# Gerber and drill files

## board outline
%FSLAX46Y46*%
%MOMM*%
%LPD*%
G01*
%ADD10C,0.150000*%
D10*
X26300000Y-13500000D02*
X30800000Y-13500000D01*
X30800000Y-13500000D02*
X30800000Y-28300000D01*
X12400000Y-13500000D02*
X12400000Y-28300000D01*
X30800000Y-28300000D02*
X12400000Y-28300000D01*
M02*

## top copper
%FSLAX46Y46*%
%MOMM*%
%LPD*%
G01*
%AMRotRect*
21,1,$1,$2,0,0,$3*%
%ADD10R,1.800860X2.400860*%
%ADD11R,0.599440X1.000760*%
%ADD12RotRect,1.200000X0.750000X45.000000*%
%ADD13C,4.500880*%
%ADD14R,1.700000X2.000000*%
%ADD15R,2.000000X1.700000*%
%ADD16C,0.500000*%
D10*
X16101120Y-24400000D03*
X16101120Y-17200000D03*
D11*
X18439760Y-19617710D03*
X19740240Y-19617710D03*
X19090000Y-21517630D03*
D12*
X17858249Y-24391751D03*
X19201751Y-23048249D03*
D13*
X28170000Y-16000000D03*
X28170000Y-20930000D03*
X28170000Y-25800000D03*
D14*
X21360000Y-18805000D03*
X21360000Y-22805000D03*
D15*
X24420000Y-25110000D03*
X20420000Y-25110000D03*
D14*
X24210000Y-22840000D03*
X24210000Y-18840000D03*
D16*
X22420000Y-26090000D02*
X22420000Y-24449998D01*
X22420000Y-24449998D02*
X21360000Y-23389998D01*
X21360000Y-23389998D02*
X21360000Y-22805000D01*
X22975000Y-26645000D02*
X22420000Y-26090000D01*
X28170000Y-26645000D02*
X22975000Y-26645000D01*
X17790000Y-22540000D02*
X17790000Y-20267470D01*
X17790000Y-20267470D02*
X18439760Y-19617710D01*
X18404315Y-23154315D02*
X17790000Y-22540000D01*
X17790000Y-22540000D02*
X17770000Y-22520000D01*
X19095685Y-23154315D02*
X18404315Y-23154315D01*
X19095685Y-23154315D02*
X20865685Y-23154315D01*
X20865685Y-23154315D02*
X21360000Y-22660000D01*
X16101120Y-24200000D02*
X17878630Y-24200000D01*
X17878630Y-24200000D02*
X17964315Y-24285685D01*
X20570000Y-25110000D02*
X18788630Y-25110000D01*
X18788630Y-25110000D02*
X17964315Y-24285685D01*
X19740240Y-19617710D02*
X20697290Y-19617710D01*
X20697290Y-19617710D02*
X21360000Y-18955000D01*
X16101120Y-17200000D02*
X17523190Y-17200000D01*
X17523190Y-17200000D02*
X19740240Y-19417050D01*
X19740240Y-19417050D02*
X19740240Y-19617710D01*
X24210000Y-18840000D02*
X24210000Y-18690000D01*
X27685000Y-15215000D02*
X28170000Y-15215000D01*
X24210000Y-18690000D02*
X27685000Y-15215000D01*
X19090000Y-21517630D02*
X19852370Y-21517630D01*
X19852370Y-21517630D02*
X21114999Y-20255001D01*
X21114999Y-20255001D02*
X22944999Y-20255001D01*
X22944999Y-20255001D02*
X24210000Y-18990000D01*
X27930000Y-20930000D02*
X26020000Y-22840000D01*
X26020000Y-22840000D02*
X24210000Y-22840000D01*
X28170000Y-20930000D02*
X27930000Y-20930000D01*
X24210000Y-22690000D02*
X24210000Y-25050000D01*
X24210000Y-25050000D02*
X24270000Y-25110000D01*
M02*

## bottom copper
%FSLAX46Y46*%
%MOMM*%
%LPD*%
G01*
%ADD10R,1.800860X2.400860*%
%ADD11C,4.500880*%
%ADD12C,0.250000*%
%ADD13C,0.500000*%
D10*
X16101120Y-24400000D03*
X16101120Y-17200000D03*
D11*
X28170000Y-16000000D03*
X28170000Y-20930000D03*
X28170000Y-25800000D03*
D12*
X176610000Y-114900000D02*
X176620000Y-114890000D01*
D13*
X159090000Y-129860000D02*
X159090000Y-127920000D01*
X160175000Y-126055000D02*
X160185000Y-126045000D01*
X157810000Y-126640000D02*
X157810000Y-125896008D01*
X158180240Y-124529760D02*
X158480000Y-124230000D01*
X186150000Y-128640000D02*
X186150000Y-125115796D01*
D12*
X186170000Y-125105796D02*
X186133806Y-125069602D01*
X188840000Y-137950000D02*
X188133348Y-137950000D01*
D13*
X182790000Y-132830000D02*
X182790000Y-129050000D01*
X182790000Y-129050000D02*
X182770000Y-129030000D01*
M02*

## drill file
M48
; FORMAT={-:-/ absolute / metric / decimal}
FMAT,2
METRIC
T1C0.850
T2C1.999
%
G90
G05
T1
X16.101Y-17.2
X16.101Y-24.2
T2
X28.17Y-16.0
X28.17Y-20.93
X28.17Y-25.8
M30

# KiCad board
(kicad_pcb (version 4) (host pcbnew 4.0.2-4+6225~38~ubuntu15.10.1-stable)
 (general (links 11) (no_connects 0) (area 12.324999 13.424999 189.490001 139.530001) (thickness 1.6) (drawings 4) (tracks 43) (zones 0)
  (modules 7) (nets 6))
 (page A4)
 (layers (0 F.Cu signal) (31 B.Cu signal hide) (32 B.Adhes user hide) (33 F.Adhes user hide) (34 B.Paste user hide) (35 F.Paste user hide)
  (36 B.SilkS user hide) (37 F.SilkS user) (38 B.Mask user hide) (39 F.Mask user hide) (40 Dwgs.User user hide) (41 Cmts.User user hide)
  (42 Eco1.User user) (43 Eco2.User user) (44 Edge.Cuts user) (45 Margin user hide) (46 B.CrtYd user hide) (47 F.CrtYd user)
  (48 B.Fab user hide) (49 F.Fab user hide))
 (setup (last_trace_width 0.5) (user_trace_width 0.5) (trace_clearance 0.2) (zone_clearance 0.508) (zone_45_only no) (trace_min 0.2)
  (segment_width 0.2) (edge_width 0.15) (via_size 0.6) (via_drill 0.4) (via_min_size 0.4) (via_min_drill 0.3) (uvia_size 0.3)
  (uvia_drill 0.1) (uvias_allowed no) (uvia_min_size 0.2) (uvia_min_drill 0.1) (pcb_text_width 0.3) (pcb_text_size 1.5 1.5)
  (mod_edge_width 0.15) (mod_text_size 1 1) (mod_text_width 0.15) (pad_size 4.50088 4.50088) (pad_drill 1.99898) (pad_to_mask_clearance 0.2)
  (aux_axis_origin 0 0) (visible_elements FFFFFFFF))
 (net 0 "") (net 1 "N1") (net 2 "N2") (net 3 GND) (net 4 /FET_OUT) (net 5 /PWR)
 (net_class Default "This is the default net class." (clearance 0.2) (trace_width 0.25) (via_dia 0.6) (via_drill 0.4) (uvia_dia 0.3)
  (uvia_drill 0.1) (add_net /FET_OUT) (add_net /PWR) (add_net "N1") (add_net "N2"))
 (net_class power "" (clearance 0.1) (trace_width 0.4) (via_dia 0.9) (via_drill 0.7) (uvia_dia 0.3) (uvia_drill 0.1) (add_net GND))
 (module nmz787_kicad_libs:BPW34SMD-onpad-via (layer F.Cu) (at 16.03 20.7 90)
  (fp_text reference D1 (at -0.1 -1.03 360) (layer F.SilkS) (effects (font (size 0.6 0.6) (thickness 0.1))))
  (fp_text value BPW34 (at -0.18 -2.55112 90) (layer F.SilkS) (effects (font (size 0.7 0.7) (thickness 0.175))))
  (pad 1 thru_hole rect (at -3.5 0.07112 90) (size 2.40086 1.80086) (drill 0.85 (offset -0.2 0)) (layers *.Cu *.Mask F.SilkS) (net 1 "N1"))
  (pad 2 thru_hole rect (at 3.5 0.07112 90) (size 2.40086 1.80086) (drill 0.85) (layers *.Cu *.Mask F.SilkS) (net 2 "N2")))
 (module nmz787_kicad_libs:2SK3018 (layer F.Cu) (at 19.09 20.56767)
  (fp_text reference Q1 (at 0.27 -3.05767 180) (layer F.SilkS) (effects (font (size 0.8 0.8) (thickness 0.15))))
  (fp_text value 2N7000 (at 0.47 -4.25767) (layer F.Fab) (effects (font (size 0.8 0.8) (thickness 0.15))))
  (pad 1 smd rect (at -0.65024 -0.94996) (size 0.59944 1.00076) (layers F.Cu F.Paste F.Mask) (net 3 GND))
  (pad 2 smd rect (at 0.65024 -0.94996) (size 0.59944 1.00076) (layers F.Cu F.Paste F.Mask) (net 2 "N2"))
  (pad 3 smd rect (at 0 0.94996) (size 0.59944 1.00076) (layers F.Cu F.Paste F.Mask) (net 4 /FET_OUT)))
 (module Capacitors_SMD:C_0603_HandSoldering (layer F.Cu) (at 18.53 23.72 45)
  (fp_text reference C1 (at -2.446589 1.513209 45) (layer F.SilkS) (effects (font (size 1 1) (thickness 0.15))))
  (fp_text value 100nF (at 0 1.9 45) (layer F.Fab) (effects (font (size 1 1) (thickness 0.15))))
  (pad 1 smd rect (at -0.95 0 45) (size 1.2 0.75) (layers F.Cu F.Paste F.Mask) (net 1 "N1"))
  (pad 2 smd rect (at 0.95 0 45) (size 1.2 0.75) (layers F.Cu F.Paste F.Mask) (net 3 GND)))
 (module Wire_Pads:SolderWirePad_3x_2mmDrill (layer F.Cu) (at 28.17 20.93 270)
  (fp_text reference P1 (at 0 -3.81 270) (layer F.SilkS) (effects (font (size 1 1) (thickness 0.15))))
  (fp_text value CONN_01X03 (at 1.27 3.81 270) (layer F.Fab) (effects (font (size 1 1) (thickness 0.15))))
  (pad 2 thru_hole circle (at -4.93 0 270) (size 4.50088 4.50088) (drill 1.99898) (layers *.Cu *.Mask F.SilkS) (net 4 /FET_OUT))
  (pad 1 thru_hole circle (at 0 0 270) (size 4.50088 4.50088) (drill 1.99898) (layers *.Cu *.Mask F.SilkS) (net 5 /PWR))
  (pad 3 thru_hole circle (at 4.87 0 270) (size 4.50088 4.50088) (drill 1.99898) (layers *.Cu *.Mask F.SilkS) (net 3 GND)))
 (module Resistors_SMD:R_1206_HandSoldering (layer F.Cu) (at 21.36 20.805 270)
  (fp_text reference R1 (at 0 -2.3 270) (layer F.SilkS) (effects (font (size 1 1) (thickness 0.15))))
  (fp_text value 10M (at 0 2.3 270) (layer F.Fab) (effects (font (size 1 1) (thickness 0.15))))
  (pad 1 smd rect (at -2 0 270) (size 2 1.7) (layers F.Cu F.Paste F.Mask) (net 2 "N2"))
  (pad 2 smd rect (at 2 0 270) (size 2 1.7) (layers F.Cu F.Paste F.Mask) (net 3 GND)))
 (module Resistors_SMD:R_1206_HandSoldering (layer F.Cu) (at 22.42 25.11 180)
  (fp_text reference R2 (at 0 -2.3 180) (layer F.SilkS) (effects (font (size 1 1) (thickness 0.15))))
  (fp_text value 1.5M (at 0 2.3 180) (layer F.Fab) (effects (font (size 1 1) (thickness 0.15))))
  (pad 1 smd rect (at -2 0 180) (size 2 1.7) (layers F.Cu F.Paste F.Mask) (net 5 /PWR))
  (pad 2 smd rect (at 2 0 180) (size 2 1.7) (layers F.Cu F.Paste F.Mask) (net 1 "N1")))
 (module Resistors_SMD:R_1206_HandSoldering (layer F.Cu) (at 24.21 20.84 90)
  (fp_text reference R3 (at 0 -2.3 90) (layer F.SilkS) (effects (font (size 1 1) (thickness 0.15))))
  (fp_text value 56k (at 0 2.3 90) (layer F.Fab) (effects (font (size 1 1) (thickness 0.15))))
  (pad 1 smd rect (at -2 0 90) (size 2 1.7) (layers F.Cu F.Paste F.Mask) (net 5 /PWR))
  (pad 2 smd rect (at 2 0 90) (size 2 1.7) (layers F.Cu F.Paste F.Mask) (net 4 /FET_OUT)))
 (gr_line (start 26.3 13.5) (end 30.8 13.5) (layer Edge.Cuts) (width 0.15))
 (gr_line (start 30.8 13.5) (end 30.8 28.3) (layer Edge.Cuts) (width 0.15))
 (gr_line (start 12.4 13.5) (end 12.4 28.3) (layer Edge.Cuts) (width 0.15))
 (gr_line (start 30.8 28.3) (end 12.4 28.3) (layer Edge.Cuts) (width 0.15))
 (segment (start 176.61 114.9) (end 176.62 114.89) (width 0.25) (layer B.Cu) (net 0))
 (segment (start 159.09 129.86) (end 159.09 127.92) (width 0.5) (layer B.Cu) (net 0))
 (segment (start 160.175 126.055) (end 160.185 126.045) (width 0.5) (layer B.Cu) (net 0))
 (segment (start 157.81 126.64) (end 157.81 125.896008) (width 0.5) (layer B.Cu) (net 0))
 (segment (start 158.18024 124.52976) (end 158.48 124.23) (width 0.5) (layer B.Cu) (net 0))
 (segment (start 186.15 128.64) (end 186.15 125.115796) (width 0.5) (layer B.Cu) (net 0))
 (segment (start 186.17 125.105796) (end 186.133806 125.069602) (width 0.25) (layer B.Cu) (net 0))
 (segment (start 188.84 137.95) (end 188.133348 137.95) (width 0.25) (layer B.Cu) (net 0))
 (segment (start 182.79 132.83) (end 182.79 129.05) (width 0.5) (layer B.Cu) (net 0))
 (segment (start 182.79 129.05) (end 182.77 129.03) (width 0.5) (layer B.Cu) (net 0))
 (segment (start 22.42 26.09) (end 22.42 24.449998) (width 0.5) (layer F.Cu) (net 3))
 (segment (start 22.42 24.449998) (end 21.36 23.389998) (width 0.5) (layer F.Cu) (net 3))
 (segment (start 21.36 23.389998) (end 21.36 22.805) (width 0.5) (layer F.Cu) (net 3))
 (segment (start 22.975 26.645) (end 22.42 26.09) (width 0.5) (layer F.Cu) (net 3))
 (segment (start 28.17 26.645) (end 22.975 26.645) (width 0.5) (layer F.Cu) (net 3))
 (segment (start 17.79 22.54) (end 17.79 20.26747) (width 0.5) (layer F.Cu) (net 3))
 (segment (start 17.79 20.26747) (end 18.43976 19.61771) (width 0.5) (layer F.Cu) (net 3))
 (segment (start 18.404315 23.154315) (end 17.79 22.54) (width 0.5) (layer F.Cu) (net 3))
 (segment (start 17.79 22.54) (end 17.77 22.52) (width 0.5) (layer F.Cu) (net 3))
 (segment (start 19.095685 23.154315) (end 18.404315 23.154315) (width 0.5) (layer F.Cu) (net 3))
 (segment (start 19.095685 23.154315) (end 20.865685 23.154315) (width 0.5) (layer F.Cu) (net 3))
 (segment (start 20.865685 23.154315) (end 21.36 22.66) (width 0.5) (layer F.Cu) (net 3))
 (segment (start 16.10112 24.2) (end 17.87863 24.2) (width 0.5) (layer F.Cu) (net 1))
 (segment (start 17.87863 24.2) (end 17.964315 24.285685) (width 0.5) (layer F.Cu) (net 1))
 (segment (start 20.57 25.11) (end 18.78863 25.11) (width 0.5) (layer F.Cu) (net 1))
 (segment (start 18.78863 25.11) (end 17.964315 24.285685) (width 0.5) (layer F.Cu) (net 1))
 (segment (start 19.74024 19.61771) (end 20.69729 19.61771) (width 0.5) (layer F.Cu) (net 2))
 (segment (start 20.69729 19.61771) (end 21.36 18.955) (width 0.5) (layer F.Cu) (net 2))
 (segment (start 16.10112 17.2) (end 17.52319 17.2) (width 0.5) (layer F.Cu) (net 2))
 (segment (start 17.52319 17.2) (end 19.74024 19.41705) (width 0.5) (layer F.Cu) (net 2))
 (segment (start 19.74024 19.41705) (end 19.74024 19.61771) (width 0.5) (layer F.Cu) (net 2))
 (segment (start 24.21 18.84) (end 24.21 18.69) (width 0.5) (layer F.Cu) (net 4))
 (segment (start 27.685 15.215) (end 28.17 15.215) (width 0.5) (layer F.Cu) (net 4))
 (segment (start 24.21 18.69) (end 27.685 15.215) (width 0.5) (layer F.Cu) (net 4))
 (segment (start 19.09 21.51763) (end 19.85237 21.51763) (width 0.5) (layer F.Cu) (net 4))
 (segment (start 19.85237 21.51763) (end 21.114999 20.255001) (width 0.5) (layer F.Cu) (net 4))
 (segment (start 21.114999 20.255001) (end 22.944999 20.255001) (width 0.5) (layer F.Cu) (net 4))
 (segment (start 22.944999 20.255001) (end 24.21 18.99) (width 0.5) (layer F.Cu) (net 4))
 (segment (start 27.93 20.93) (end 26.02 22.84) (width 0.5) (layer F.Cu) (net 5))
 (segment (start 26.02 22.84) (end 24.21 22.84) (width 0.5) (layer F.Cu) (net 5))
 (segment (start 28.17 20.93) (end 27.93 20.93) (width 0.5) (layer F.Cu) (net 5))
 (segment (start 24.21 22.69) (end 24.21 25.05) (width 0.5) (layer F.Cu) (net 5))
 (segment (start 24.21 25.05) (end 24.27 25.11) (width 0.5) (layer F.Cu) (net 5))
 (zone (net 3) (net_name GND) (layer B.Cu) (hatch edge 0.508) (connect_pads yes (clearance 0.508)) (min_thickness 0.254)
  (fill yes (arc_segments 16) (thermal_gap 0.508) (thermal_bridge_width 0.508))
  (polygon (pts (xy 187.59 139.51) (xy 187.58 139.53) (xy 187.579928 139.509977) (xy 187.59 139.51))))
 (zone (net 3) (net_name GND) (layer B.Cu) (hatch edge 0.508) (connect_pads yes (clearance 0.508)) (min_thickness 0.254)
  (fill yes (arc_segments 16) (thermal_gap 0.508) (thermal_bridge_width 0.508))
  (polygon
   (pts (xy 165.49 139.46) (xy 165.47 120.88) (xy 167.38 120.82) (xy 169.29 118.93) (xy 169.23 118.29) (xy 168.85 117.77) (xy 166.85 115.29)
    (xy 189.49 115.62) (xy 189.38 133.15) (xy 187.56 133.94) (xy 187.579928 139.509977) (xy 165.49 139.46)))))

